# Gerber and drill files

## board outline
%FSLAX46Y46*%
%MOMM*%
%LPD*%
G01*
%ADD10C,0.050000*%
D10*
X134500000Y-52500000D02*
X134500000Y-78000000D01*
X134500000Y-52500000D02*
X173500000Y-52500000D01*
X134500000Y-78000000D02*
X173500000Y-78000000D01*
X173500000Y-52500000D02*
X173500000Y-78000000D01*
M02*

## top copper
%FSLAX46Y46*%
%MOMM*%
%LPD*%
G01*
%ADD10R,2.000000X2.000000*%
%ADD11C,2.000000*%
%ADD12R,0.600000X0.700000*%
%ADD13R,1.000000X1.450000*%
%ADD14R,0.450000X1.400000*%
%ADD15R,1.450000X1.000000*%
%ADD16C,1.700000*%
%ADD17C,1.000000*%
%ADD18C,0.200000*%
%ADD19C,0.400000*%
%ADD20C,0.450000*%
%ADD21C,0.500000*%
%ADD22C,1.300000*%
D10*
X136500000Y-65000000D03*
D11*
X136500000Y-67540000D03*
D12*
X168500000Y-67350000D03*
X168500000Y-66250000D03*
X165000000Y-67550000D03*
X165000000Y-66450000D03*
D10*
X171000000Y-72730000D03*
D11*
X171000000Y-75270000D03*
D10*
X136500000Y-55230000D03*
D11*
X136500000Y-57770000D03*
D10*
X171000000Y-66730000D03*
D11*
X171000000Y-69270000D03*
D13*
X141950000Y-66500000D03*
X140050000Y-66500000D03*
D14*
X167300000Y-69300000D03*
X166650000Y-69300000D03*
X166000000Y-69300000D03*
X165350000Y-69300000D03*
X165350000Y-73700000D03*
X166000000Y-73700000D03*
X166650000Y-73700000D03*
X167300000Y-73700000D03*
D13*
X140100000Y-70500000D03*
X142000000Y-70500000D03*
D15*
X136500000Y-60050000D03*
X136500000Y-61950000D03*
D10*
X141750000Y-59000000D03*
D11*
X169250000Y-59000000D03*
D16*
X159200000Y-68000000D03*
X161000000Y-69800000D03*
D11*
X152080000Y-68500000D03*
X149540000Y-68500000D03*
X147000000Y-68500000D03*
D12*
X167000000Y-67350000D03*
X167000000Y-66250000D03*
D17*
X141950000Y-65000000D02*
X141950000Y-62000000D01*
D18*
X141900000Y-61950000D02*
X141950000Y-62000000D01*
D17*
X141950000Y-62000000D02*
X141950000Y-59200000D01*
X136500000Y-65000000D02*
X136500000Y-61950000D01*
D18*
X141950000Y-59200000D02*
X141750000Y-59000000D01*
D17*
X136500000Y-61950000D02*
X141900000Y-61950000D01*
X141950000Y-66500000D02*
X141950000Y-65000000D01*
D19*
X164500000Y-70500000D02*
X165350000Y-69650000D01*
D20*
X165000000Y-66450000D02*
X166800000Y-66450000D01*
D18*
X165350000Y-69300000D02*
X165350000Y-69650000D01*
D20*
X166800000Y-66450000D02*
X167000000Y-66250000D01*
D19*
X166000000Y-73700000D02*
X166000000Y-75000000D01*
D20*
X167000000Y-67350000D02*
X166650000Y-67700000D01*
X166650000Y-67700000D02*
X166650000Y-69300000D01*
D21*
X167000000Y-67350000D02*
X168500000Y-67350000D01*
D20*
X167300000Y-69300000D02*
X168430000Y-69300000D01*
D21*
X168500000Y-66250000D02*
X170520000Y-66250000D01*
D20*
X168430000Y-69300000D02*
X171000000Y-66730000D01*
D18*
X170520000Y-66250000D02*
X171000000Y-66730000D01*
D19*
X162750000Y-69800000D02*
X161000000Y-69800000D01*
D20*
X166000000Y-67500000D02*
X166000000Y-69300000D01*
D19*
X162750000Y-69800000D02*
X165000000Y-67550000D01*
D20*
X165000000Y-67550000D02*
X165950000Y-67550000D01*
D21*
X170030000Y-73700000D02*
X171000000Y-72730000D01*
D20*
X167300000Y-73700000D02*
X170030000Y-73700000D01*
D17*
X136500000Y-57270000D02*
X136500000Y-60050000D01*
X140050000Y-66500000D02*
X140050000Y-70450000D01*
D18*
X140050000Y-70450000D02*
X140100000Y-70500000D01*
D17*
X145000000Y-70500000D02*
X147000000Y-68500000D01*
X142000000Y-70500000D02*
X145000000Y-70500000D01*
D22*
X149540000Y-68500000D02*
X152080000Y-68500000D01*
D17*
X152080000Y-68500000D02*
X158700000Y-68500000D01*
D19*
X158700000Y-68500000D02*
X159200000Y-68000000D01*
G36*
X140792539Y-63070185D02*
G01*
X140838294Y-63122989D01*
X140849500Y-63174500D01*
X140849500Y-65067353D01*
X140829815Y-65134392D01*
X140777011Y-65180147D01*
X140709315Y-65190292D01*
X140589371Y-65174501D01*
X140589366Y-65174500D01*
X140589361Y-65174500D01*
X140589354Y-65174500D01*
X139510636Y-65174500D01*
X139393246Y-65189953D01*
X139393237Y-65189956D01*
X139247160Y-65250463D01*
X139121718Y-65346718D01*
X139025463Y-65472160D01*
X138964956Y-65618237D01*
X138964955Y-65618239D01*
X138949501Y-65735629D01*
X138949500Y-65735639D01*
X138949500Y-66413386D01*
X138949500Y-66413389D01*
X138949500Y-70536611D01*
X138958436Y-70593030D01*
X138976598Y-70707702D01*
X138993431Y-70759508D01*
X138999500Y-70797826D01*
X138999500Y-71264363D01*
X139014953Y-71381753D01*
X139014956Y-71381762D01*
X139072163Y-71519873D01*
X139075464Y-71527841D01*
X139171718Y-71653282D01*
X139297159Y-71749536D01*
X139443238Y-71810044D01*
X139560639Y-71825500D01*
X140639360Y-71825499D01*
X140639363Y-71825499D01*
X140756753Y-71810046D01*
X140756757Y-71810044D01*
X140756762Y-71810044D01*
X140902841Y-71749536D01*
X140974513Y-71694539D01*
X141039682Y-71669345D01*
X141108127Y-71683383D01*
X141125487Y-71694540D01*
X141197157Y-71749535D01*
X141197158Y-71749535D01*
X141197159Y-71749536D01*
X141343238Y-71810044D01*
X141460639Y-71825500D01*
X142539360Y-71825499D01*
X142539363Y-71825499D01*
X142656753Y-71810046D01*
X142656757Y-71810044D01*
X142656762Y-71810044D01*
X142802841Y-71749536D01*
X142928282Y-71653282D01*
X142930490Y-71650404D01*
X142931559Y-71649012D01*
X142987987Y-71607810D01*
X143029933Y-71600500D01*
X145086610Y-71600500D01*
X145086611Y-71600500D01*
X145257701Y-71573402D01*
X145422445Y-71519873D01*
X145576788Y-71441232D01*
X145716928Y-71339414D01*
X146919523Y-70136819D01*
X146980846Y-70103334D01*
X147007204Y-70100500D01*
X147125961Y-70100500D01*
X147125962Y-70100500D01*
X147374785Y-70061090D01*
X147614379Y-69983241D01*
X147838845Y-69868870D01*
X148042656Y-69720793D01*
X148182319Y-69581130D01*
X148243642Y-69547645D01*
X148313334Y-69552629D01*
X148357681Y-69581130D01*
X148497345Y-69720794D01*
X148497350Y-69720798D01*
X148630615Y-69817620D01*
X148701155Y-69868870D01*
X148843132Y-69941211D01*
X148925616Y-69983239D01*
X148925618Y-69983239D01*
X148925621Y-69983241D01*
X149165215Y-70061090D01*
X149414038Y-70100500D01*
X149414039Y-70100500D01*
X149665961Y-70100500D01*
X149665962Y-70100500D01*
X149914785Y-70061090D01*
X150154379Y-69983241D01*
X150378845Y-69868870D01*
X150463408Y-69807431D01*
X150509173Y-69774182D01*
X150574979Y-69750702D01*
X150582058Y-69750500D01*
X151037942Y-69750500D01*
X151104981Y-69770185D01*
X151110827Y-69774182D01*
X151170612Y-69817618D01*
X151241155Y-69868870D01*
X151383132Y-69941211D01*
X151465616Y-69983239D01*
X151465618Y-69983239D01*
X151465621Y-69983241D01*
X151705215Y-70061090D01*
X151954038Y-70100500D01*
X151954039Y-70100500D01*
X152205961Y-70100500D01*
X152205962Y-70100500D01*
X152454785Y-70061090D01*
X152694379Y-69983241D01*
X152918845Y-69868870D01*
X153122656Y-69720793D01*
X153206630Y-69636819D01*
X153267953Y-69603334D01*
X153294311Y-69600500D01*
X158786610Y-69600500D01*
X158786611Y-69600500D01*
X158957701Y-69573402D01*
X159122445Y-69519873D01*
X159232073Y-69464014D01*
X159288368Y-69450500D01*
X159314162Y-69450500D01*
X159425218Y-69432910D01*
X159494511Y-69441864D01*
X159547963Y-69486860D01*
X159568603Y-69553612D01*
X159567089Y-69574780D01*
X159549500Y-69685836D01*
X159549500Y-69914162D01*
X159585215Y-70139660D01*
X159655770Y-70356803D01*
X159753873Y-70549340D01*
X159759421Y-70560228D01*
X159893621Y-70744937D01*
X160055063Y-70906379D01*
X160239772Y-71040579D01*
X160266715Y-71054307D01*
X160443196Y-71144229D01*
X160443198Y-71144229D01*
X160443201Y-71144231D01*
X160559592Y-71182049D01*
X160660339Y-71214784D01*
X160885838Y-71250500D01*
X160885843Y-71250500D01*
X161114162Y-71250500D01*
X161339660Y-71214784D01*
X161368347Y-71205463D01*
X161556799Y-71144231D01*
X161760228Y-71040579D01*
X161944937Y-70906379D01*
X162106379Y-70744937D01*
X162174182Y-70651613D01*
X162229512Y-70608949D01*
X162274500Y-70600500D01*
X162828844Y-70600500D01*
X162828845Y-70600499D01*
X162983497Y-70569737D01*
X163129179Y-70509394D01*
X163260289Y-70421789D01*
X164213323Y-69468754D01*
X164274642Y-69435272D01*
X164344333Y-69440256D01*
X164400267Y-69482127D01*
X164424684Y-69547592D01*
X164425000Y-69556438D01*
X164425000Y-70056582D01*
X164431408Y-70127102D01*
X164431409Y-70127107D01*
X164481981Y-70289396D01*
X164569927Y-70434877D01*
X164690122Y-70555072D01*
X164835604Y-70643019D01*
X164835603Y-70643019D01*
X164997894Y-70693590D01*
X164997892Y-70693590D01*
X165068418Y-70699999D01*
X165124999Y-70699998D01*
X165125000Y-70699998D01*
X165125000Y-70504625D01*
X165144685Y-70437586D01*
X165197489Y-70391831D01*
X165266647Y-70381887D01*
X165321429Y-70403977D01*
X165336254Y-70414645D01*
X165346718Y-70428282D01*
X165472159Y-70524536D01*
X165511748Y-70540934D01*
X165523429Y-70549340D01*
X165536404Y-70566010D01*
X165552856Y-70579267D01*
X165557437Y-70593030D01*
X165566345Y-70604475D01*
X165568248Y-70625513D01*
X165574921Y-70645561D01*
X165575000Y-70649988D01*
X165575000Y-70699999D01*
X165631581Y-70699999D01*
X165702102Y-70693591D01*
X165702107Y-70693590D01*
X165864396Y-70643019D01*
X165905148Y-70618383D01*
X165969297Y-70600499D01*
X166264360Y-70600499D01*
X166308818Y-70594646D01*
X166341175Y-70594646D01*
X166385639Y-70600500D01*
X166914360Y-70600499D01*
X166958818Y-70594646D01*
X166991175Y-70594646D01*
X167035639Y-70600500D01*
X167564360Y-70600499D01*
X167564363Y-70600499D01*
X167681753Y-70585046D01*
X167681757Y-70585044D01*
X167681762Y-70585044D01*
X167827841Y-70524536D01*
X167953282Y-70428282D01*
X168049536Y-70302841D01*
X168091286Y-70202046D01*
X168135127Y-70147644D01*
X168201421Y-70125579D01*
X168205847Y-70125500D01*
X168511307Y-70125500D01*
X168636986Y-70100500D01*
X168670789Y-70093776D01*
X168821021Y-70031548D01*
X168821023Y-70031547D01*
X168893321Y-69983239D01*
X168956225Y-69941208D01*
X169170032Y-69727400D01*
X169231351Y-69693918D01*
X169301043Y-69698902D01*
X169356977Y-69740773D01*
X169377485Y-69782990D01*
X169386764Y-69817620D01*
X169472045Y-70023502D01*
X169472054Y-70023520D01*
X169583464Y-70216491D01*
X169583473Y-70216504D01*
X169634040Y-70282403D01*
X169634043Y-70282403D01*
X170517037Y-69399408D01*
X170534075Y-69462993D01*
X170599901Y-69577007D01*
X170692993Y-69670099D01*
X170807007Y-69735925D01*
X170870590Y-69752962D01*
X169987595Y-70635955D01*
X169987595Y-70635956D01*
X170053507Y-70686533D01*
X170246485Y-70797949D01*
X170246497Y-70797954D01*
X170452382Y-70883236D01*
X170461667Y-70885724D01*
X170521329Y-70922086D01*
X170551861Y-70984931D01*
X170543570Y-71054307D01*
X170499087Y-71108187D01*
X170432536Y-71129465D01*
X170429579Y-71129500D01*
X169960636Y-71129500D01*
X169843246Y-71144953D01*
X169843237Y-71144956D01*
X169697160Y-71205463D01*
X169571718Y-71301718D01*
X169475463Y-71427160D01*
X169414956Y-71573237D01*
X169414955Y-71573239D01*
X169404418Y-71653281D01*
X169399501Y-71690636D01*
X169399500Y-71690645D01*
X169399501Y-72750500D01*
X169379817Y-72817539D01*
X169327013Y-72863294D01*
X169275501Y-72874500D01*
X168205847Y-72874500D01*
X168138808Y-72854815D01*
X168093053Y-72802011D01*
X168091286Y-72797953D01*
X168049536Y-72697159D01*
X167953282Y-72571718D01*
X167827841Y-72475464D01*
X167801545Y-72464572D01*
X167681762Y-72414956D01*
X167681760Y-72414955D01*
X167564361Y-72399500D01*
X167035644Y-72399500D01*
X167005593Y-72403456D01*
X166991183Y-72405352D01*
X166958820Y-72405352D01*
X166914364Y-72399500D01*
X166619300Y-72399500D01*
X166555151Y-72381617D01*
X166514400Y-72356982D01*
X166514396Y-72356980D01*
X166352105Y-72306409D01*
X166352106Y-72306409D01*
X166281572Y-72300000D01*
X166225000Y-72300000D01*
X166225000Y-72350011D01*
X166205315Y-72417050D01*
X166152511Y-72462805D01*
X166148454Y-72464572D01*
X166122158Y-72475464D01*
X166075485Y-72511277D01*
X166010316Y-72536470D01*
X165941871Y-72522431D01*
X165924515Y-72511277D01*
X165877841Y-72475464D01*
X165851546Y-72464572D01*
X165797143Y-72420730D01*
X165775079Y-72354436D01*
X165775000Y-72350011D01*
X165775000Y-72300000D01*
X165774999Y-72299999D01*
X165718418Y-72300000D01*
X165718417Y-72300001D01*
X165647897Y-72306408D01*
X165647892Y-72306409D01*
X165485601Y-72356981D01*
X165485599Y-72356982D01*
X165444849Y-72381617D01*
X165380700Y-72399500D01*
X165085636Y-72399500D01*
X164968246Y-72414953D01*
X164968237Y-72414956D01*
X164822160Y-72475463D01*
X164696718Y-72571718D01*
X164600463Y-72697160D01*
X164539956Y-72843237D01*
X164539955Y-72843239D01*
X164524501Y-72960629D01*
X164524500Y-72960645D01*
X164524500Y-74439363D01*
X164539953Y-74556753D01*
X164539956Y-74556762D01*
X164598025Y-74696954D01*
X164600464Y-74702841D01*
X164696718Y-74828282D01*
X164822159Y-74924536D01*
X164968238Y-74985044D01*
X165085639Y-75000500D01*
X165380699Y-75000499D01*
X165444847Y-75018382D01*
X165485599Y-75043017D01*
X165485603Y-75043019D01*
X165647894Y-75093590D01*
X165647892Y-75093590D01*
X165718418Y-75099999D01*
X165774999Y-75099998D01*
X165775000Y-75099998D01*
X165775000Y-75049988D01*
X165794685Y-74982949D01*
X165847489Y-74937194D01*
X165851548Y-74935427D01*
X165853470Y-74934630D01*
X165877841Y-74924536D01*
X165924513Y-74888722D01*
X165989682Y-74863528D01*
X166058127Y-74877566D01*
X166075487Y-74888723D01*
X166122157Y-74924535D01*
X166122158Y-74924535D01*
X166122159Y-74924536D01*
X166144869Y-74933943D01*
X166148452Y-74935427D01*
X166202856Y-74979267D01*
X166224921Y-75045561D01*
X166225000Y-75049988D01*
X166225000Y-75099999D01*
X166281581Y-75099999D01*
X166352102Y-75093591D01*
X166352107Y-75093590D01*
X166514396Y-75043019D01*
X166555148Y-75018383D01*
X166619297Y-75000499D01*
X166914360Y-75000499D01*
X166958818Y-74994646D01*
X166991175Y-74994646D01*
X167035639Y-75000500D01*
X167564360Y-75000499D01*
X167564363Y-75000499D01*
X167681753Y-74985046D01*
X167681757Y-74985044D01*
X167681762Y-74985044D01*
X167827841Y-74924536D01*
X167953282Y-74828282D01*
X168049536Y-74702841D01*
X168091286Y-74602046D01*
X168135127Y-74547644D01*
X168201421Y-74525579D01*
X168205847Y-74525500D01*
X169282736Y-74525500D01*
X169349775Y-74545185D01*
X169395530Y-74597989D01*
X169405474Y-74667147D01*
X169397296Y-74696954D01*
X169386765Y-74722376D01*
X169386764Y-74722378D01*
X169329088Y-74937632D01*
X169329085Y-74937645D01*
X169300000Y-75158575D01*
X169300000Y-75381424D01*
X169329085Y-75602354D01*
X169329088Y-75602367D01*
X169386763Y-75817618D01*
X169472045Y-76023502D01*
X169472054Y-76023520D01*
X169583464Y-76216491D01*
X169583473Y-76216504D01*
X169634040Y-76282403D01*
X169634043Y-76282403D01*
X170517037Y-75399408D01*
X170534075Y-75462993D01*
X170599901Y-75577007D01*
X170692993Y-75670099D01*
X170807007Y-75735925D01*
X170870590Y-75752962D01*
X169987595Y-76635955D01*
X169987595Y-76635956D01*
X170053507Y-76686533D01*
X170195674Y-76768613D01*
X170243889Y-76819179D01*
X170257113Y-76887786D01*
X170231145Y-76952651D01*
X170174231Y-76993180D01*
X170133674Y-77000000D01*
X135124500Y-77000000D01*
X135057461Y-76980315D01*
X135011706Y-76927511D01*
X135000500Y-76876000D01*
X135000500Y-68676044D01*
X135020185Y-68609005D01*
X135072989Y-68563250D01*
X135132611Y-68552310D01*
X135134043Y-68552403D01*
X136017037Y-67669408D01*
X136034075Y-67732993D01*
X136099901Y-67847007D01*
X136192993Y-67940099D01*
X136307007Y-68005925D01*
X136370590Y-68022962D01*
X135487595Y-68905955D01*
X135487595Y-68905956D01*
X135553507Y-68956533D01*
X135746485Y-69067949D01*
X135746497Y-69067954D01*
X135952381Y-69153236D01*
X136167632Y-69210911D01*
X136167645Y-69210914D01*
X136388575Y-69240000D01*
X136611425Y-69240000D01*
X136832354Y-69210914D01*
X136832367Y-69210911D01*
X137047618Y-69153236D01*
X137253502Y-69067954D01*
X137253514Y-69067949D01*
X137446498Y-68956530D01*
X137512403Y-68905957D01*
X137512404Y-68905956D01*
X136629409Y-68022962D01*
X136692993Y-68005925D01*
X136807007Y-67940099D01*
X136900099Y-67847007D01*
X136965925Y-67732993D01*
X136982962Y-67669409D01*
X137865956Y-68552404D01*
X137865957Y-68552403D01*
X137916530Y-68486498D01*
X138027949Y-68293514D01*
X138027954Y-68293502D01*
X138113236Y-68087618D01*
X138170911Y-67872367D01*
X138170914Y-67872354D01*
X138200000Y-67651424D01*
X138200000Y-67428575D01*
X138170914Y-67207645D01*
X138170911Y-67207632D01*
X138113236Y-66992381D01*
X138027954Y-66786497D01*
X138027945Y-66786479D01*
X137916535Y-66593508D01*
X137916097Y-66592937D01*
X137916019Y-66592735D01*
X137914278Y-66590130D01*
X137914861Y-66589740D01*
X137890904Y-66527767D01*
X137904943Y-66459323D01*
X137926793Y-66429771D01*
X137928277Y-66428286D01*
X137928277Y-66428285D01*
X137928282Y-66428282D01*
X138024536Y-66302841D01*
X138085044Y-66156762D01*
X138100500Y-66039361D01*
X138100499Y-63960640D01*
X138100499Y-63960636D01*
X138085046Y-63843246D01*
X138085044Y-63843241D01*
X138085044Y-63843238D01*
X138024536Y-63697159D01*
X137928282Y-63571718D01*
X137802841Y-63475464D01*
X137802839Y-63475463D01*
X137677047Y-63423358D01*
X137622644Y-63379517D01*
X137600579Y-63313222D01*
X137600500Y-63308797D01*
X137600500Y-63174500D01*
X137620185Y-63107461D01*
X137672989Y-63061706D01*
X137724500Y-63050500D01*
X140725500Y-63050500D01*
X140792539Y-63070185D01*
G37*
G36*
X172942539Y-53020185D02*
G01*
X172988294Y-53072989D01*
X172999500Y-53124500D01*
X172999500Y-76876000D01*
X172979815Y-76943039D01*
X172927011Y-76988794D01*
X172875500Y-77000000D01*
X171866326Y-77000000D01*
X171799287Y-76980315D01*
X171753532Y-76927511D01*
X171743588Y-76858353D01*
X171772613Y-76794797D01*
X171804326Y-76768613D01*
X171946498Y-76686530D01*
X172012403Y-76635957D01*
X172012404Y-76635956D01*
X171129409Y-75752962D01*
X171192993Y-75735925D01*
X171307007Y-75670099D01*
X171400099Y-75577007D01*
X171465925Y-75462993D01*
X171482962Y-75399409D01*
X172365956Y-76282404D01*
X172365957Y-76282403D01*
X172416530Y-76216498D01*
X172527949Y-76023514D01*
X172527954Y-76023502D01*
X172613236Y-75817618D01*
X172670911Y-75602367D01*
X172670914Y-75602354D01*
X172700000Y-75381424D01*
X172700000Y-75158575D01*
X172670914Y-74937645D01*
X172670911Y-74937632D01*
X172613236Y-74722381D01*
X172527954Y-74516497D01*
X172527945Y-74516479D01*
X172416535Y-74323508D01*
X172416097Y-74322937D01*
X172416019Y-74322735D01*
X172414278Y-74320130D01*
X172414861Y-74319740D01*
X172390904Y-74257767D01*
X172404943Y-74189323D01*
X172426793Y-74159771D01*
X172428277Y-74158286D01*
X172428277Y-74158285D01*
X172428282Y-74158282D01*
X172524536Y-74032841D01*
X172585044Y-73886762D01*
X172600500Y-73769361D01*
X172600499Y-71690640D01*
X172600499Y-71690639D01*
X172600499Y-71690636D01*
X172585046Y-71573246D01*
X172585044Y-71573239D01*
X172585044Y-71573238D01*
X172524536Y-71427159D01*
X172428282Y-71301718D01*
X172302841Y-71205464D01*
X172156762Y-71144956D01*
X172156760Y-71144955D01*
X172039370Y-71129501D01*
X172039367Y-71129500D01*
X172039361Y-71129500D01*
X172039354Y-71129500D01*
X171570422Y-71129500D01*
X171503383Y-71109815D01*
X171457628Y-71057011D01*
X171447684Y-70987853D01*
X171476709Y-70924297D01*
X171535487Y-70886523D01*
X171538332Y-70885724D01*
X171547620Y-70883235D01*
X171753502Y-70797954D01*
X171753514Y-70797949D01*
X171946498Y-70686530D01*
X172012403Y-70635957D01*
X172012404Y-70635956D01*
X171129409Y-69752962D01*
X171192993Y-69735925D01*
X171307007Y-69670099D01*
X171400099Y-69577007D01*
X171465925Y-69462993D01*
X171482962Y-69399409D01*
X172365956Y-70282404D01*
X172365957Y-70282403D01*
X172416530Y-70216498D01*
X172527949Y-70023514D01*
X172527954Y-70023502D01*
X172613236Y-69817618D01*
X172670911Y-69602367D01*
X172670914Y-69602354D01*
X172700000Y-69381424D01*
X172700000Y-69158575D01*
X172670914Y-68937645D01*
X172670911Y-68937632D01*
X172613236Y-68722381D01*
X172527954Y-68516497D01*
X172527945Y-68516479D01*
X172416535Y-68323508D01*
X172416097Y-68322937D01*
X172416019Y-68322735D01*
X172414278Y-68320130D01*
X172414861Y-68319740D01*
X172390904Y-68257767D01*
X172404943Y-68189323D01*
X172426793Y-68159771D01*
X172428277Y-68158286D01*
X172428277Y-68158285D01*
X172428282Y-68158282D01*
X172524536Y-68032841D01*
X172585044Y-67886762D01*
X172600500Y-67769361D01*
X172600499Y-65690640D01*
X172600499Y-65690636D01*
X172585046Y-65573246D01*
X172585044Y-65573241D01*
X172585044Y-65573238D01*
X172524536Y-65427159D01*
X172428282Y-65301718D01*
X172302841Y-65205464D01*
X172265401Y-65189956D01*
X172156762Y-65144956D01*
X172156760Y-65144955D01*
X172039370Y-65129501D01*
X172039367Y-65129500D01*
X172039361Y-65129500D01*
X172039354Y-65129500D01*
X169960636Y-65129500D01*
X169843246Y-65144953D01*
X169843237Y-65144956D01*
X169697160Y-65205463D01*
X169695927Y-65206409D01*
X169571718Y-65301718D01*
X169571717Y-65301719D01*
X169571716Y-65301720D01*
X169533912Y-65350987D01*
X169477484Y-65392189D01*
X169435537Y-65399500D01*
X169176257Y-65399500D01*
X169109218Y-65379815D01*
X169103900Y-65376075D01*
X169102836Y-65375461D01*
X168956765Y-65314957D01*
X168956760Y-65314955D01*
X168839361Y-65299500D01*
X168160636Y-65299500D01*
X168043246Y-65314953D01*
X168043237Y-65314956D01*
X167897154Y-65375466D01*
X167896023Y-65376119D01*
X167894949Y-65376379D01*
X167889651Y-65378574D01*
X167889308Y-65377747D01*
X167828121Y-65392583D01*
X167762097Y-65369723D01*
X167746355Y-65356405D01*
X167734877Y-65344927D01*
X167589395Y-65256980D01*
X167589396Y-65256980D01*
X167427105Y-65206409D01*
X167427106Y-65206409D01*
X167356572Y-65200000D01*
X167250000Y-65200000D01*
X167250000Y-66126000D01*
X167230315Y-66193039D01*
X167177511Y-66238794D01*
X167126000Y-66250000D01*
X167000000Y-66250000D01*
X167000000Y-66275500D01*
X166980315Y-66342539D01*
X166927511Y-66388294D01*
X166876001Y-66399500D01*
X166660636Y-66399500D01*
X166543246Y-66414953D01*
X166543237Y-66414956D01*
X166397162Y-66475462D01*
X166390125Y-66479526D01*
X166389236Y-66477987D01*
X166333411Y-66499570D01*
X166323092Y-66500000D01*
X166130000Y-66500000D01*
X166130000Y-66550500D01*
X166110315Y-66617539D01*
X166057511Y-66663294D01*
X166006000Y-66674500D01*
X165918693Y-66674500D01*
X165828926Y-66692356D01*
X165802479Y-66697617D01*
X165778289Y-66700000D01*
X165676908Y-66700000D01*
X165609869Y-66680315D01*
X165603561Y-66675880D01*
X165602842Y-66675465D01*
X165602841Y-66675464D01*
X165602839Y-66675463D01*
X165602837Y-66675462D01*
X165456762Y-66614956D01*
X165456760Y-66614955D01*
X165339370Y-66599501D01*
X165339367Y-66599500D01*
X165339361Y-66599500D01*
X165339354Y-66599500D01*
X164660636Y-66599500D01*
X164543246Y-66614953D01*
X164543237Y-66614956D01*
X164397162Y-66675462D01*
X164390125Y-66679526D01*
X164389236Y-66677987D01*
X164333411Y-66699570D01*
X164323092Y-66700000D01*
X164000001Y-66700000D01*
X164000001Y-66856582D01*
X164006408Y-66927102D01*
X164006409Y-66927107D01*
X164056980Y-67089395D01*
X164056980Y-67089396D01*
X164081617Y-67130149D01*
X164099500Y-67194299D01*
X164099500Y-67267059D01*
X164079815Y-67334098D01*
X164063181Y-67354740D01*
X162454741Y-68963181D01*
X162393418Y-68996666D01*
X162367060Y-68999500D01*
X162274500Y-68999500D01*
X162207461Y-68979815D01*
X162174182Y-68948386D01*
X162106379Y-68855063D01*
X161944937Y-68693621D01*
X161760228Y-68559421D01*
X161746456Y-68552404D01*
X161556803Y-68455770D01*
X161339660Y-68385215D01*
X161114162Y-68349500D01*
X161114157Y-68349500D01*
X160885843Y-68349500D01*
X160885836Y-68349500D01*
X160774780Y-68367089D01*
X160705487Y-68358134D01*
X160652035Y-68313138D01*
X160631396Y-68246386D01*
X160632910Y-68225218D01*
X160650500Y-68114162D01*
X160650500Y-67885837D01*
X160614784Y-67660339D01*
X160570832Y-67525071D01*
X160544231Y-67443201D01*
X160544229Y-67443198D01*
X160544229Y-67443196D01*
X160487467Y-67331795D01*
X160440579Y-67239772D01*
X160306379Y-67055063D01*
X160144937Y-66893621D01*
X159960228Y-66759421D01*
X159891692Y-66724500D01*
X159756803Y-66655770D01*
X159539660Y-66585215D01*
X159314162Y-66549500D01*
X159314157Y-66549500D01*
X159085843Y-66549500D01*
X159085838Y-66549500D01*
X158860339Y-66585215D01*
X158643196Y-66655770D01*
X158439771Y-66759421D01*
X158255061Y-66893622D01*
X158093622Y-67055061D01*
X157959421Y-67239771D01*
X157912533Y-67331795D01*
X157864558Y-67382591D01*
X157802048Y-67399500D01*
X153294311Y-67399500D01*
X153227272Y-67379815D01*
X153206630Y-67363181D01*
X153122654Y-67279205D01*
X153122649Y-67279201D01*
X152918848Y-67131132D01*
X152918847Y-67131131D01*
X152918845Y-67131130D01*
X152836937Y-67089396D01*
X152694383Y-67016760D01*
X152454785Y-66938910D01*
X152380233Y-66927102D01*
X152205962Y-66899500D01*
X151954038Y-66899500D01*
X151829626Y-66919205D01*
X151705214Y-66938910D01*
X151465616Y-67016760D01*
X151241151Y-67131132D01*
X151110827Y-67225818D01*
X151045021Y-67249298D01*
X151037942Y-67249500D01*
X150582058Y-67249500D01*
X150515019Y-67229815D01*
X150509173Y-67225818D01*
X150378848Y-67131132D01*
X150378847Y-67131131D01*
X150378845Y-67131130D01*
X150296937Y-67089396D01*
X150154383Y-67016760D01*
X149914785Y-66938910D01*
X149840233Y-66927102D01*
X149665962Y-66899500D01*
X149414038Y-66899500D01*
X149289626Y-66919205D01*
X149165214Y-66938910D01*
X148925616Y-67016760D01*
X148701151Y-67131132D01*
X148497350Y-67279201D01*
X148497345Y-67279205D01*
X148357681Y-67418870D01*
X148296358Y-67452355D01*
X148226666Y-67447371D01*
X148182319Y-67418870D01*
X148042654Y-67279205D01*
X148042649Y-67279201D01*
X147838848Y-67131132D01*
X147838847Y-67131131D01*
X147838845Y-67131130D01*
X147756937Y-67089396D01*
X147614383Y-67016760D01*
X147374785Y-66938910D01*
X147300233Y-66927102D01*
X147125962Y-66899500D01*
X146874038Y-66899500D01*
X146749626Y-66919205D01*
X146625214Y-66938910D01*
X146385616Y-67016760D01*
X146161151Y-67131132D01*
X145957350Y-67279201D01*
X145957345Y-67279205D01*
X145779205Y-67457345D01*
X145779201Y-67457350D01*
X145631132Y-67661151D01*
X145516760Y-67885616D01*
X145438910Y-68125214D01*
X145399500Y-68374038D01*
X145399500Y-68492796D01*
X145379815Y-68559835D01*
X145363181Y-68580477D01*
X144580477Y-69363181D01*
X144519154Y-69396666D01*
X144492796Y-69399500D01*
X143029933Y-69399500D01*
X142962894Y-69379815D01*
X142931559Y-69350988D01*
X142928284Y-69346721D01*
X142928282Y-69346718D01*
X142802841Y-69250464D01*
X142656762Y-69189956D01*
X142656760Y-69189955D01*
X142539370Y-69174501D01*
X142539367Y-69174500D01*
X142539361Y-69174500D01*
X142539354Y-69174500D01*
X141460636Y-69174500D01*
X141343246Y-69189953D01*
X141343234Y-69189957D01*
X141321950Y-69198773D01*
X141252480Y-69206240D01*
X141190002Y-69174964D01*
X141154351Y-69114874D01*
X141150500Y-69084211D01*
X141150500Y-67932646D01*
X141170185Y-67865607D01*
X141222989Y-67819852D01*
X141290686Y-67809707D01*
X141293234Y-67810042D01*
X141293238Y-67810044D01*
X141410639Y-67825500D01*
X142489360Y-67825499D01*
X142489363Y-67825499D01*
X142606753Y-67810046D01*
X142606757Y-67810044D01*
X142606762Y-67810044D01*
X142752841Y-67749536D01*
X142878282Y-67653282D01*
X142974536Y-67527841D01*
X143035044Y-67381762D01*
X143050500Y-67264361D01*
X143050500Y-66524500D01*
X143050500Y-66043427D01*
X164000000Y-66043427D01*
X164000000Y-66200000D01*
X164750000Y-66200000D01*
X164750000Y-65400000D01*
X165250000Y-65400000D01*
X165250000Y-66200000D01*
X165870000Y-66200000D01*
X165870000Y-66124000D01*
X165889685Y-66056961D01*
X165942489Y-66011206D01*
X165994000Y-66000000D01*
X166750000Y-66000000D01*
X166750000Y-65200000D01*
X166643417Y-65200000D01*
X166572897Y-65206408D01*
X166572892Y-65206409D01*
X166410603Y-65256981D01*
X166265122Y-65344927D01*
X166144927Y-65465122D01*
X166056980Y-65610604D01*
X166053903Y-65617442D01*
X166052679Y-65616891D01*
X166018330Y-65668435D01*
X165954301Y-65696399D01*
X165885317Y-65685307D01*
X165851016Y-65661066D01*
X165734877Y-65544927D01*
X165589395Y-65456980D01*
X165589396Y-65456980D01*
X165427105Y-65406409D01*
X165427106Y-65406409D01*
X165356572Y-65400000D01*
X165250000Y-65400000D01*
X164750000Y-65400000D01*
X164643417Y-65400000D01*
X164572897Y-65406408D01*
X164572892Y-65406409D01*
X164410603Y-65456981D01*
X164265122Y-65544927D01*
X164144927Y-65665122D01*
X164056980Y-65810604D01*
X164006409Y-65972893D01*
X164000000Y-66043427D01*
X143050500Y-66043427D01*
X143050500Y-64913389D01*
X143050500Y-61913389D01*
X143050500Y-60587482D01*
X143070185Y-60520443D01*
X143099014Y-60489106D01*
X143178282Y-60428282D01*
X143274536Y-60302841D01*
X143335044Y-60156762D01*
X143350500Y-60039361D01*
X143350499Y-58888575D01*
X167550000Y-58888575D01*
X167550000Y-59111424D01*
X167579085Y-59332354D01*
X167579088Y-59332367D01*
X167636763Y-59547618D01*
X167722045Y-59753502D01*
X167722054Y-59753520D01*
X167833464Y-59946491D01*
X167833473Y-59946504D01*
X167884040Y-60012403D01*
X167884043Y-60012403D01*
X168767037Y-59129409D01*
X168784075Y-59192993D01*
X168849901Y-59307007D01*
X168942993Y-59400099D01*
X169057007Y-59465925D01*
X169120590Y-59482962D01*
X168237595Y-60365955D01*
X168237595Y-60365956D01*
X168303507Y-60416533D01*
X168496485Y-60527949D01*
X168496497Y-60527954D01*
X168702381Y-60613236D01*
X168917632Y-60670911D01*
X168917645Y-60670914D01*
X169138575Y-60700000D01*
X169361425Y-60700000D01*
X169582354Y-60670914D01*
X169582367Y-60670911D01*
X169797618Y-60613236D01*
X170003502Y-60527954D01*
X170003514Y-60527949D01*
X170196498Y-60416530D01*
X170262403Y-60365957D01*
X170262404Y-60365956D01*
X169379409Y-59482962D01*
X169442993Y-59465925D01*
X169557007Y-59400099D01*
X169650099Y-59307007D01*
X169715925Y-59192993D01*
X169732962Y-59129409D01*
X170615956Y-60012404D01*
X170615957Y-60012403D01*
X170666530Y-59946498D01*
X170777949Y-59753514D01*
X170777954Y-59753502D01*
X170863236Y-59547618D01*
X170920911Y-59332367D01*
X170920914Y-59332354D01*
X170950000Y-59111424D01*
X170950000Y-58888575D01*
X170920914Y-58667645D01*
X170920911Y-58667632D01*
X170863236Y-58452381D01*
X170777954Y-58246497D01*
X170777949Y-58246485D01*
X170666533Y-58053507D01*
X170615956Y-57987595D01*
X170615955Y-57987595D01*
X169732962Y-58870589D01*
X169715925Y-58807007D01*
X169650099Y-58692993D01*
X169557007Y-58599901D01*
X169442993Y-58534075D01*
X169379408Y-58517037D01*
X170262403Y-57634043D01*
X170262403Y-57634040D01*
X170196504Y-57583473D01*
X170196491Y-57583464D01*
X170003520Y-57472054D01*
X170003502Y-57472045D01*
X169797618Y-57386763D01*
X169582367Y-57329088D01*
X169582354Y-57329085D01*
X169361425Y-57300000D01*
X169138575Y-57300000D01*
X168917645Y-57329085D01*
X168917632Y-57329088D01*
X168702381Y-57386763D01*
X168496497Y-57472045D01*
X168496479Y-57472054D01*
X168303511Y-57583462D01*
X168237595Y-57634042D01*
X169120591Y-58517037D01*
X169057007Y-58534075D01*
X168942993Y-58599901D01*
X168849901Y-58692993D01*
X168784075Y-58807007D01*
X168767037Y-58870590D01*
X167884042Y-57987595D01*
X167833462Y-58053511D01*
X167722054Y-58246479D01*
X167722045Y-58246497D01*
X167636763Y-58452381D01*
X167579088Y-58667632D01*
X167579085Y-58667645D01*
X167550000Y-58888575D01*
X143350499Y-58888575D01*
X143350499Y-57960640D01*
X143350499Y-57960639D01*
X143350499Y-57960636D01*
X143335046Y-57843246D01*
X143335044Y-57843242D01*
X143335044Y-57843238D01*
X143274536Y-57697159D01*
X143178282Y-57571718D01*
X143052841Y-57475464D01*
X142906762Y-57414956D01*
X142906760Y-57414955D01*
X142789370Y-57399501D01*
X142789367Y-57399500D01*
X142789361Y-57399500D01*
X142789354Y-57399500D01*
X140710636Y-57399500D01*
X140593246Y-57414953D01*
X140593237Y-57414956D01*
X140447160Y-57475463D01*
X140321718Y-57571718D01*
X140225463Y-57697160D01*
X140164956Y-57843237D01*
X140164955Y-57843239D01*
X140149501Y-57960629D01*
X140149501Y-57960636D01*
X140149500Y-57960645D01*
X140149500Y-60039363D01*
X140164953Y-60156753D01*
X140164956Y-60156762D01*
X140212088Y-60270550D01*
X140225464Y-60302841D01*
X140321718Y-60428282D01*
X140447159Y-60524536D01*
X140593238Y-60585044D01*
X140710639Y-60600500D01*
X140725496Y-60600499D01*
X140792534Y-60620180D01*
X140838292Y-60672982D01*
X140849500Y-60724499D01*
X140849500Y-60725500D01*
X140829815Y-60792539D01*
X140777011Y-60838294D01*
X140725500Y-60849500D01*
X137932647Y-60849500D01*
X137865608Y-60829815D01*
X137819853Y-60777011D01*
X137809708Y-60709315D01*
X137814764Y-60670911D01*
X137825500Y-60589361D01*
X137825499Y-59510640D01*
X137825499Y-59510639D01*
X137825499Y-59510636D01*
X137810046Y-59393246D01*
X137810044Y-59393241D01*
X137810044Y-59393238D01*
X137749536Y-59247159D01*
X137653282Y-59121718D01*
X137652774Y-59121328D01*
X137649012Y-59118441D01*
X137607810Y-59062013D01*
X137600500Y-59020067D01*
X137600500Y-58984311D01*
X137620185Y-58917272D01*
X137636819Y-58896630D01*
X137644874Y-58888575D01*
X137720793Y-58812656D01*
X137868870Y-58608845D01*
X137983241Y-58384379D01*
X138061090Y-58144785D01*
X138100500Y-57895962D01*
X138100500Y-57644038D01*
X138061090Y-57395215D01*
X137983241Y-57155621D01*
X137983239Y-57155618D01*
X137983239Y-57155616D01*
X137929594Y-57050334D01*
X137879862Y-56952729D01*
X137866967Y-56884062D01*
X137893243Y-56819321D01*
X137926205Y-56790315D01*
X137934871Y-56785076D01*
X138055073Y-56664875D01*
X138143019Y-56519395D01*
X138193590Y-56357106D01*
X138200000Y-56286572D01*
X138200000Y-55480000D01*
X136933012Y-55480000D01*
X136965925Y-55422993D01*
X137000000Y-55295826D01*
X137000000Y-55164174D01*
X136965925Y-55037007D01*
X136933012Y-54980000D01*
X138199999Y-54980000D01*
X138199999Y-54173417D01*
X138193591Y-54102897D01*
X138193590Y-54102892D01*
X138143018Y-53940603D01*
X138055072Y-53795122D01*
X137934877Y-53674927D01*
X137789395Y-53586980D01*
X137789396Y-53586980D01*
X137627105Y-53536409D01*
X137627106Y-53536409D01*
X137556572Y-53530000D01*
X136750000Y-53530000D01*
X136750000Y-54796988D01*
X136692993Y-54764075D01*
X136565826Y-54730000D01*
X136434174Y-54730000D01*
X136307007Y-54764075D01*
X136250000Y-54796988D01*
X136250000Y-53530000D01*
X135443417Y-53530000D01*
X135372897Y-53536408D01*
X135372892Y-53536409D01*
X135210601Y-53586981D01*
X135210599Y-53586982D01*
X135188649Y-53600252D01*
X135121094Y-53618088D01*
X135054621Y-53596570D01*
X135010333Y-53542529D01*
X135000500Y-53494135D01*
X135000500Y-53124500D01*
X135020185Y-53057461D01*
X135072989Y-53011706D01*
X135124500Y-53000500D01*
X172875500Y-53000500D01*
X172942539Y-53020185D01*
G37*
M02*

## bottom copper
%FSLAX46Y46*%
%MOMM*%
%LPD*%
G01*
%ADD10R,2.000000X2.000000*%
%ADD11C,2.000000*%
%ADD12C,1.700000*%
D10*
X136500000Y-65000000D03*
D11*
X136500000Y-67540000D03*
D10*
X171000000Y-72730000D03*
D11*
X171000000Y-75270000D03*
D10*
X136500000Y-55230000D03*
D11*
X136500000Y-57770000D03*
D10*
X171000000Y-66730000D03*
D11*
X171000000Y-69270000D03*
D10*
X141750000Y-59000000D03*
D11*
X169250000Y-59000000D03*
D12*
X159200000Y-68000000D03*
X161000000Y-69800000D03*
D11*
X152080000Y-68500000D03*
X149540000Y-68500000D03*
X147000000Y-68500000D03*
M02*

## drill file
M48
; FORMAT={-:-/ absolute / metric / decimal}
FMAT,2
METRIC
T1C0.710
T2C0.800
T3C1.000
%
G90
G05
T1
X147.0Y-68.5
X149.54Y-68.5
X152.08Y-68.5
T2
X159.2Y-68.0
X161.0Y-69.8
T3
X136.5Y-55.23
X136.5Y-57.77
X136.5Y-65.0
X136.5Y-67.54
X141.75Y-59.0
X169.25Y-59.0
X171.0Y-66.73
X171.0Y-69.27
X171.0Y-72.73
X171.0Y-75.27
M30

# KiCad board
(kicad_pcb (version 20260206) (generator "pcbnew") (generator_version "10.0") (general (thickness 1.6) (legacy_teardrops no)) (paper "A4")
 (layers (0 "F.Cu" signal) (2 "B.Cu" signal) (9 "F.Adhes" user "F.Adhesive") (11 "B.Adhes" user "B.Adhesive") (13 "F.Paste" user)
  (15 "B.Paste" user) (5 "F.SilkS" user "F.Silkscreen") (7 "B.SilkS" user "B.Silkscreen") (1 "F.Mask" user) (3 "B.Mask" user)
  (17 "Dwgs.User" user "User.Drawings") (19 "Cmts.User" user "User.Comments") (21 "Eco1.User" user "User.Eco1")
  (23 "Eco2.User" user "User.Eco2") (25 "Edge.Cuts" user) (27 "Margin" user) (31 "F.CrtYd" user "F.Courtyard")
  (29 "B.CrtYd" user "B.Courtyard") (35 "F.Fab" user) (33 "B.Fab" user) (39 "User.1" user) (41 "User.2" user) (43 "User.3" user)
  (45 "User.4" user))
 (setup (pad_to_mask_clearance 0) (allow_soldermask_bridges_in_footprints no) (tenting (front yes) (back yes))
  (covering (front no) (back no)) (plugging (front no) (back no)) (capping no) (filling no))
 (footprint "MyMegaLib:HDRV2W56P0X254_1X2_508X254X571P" (layer "F.Cu") (at 136.5 65 -90)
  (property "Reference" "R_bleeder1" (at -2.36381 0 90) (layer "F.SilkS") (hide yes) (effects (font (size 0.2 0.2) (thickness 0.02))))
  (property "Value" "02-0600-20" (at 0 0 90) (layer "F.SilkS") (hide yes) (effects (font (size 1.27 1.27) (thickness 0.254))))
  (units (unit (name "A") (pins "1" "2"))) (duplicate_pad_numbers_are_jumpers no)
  (pad "1" thru_hole rect (at 0 0 270) (size 2 2) (drill 1) (layers "*.Cu" "*.Mask") (remove_unused_layers no)
   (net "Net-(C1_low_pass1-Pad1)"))
  (pad "2" thru_hole circle (at 2.54 0 270) (size 2 2) (drill 1) (layers "*.Cu" "*.Mask") (remove_unused_layers no) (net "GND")))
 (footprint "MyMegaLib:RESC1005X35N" (layer "F.Cu") (at 168.5 66.8 90)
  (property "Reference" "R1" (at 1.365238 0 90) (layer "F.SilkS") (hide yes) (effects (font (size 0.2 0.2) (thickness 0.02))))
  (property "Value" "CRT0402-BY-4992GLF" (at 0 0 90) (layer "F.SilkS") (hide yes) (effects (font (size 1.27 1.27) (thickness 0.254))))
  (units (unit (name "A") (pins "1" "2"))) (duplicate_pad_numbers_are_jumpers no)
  (pad "1" smd rect (at -0.55 0 180) (size 0.6 0.7) (layers "F.Cu" "F.Mask" "F.Paste") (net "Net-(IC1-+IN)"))
  (pad "2" smd rect (at 0.55 0 180) (size 0.6 0.7) (layers "F.Cu" "F.Mask" "F.Paste") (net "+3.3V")))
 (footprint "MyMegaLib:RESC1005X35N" (layer "F.Cu") (at 165 67 90)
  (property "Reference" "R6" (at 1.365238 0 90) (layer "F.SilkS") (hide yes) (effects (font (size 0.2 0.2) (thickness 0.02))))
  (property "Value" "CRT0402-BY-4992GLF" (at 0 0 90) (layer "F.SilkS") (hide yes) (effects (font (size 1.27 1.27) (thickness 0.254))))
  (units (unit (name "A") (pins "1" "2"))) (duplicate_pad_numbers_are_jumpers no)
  (pad "1" smd rect (at -0.55 0 180) (size 0.6 0.7) (layers "F.Cu" "F.Mask" "F.Paste") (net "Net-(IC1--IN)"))
  (pad "2" smd rect (at 0.55 0 180) (size 0.6 0.7) (layers "F.Cu" "F.Mask" "F.Paste") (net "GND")))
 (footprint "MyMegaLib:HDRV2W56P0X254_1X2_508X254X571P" (layer "F.Cu") (at 171 72.73 -90)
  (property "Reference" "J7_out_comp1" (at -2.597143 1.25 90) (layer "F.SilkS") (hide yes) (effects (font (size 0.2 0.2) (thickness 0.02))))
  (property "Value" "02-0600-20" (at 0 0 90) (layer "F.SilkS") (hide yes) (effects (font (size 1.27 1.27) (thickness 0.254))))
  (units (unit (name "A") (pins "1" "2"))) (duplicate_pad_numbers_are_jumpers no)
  (pad "1" thru_hole rect (at 0 0 270) (size 2 2) (drill 1) (layers "*.Cu" "*.Mask") (remove_unused_layers no) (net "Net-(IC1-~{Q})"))
  (pad "2" thru_hole circle (at 2.54 0 270) (size 2 2) (drill 1) (layers "*.Cu" "*.Mask") (remove_unused_layers no) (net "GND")))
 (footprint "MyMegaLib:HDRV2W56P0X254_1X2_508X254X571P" (layer "F.Cu") (at 136.5 55.23 -90)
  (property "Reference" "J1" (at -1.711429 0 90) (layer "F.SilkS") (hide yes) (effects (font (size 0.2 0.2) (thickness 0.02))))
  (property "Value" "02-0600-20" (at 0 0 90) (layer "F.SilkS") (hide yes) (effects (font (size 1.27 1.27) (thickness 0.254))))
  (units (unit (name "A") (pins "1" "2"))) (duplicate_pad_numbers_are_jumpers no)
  (pad "1" thru_hole rect (at 0 0 270) (size 2 2) (drill 1) (layers "*.Cu" "*.Mask") (remove_unused_layers no) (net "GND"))
  (pad "2" thru_hole circle (at 2.54 0 270) (size 2 2) (drill 1) (layers "*.Cu" "*.Mask") (remove_unused_layers no) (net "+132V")))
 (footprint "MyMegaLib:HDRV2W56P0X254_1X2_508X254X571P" (layer "F.Cu") (at 171 66.73 -90)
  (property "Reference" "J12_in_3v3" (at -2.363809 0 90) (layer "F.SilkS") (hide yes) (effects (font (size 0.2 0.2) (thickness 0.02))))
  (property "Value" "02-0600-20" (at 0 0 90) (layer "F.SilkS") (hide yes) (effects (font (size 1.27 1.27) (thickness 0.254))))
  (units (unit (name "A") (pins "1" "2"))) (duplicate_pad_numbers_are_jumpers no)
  (pad "1" thru_hole rect (at 0 0 270) (size 2 2) (drill 1) (layers "*.Cu" "*.Mask") (remove_unused_layers no) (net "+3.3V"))
  (pad "2" thru_hole circle (at 2.54 0 270) (size 2 2) (drill 1) (layers "*.Cu" "*.Mask") (remove_unused_layers no) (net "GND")))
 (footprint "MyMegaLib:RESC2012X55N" (layer "F.Cu") (at 141 66.5 180)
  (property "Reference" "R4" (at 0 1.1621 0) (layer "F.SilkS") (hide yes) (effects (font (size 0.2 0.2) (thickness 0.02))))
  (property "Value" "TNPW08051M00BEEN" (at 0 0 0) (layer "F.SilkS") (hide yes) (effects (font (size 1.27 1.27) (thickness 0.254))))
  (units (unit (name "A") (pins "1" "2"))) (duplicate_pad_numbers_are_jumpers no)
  (pad "1" smd rect (at -0.95 0 180) (size 1 1.45) (layers "F.Cu" "F.Mask" "F.Paste") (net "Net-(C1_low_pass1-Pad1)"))
  (pad "2" smd rect (at 0.95 0 180) (size 1 1.45) (layers "F.Cu" "F.Mask" "F.Paste") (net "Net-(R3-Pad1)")))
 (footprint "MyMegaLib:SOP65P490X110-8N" (layer "F.Cu") (at 166.325 71.5 -90)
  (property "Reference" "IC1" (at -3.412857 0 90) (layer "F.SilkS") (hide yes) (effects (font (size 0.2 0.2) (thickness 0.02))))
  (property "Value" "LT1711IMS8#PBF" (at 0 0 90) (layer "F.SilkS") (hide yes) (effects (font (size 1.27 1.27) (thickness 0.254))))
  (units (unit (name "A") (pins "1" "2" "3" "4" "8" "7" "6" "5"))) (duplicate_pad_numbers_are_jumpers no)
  (pad "1" smd rect (at -2.2 -0.975) (size 0.45 1.4) (layers "F.Cu" "F.Mask" "F.Paste") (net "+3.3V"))
  (pad "2" smd rect (at -2.2 -0.325) (size 0.45 1.4) (layers "F.Cu" "F.Mask" "F.Paste") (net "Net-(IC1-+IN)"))
  (pad "3" smd rect (at -2.2 0.325) (size 0.45 1.4) (layers "F.Cu" "F.Mask" "F.Paste") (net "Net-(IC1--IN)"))
  (pad "4" smd rect (at -2.2 0.975) (size 0.45 1.4) (layers "F.Cu" "F.Mask" "F.Paste") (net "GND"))
  (pad "5" smd rect (at 2.2 0.975) (size 0.45 1.4) (layers "F.Cu" "F.Mask" "F.Paste") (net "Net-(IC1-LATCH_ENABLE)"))
  (pad "6" smd rect (at 2.2 0.325) (size 0.45 1.4) (layers "F.Cu" "F.Mask" "F.Paste") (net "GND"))
  (pad "7" smd rect (at 2.2 -0.325) (size 0.45 1.4) (layers "F.Cu" "F.Mask" "F.Paste") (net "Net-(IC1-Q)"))
  (pad "8" smd rect (at 2.2 -0.975) (size 0.45 1.4) (layers "F.Cu" "F.Mask" "F.Paste") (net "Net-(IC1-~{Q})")))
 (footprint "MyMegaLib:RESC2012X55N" (layer "F.Cu") (at 141.05 70.5)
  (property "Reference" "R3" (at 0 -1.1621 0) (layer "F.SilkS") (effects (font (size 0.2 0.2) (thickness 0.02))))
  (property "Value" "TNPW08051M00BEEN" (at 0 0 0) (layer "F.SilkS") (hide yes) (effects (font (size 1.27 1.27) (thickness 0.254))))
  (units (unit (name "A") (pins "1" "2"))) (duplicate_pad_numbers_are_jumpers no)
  (pad "1" smd rect (at -0.95 0) (size 1 1.45) (layers "F.Cu" "F.Mask" "F.Paste") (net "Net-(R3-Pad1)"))
  (pad "2" smd rect (at 0.95 0) (size 1 1.45) (layers "F.Cu" "F.Mask" "F.Paste") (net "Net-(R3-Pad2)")))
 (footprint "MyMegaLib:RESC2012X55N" (layer "F.Cu") (at 136.5 61 -90)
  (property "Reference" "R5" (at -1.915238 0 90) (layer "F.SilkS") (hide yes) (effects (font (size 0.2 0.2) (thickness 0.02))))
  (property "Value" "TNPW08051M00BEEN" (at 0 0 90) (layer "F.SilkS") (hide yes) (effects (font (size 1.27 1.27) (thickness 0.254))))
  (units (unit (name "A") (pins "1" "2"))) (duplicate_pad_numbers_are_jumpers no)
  (pad "1" smd rect (at -0.95 0 270) (size 1 1.45) (layers "F.Cu" "F.Mask" "F.Paste") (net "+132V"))
  (pad "2" smd rect (at 0.95 0 270) (size 1 1.45) (layers "F.Cu" "F.Mask" "F.Paste") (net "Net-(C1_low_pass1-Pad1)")))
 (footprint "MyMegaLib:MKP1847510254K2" (layer "F.Cu") (at 141.75 59)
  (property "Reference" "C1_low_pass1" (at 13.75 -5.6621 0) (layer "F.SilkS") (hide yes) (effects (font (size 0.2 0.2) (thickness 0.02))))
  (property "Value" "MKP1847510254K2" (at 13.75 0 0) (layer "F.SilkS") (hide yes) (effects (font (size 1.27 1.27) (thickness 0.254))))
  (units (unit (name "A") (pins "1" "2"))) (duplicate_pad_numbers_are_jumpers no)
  (pad "1" thru_hole rect (at 0 0) (size 2 2) (drill 1) (layers "*.Cu" "*.Mask") (remove_unused_layers no) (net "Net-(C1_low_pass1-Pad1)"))
  (pad "2" thru_hole circle (at 27.5 0) (size 2 2) (drill 1) (layers "*.Cu" "*.Mask") (remove_unused_layers no) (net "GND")))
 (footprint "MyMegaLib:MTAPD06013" (layer "F.Cu") (at 160.1 68.9 -90)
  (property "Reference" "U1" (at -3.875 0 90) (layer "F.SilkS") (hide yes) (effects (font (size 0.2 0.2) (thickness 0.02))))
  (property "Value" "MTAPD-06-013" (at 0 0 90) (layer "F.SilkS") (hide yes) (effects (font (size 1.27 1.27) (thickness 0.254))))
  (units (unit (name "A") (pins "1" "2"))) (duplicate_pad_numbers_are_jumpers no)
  (pad "1" thru_hole circle (at -0.9 0.9 270) (size 1.7 1.7) (drill 0.8) (layers "*.Cu" "*.Mask") (remove_unused_layers no)
   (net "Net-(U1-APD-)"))
  (pad "2" thru_hole circle (at 0.9 -0.9 270) (size 1.7 1.7) (drill 0.8) (layers "*.Cu" "*.Mask") (remove_unused_layers no)
   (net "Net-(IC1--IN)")))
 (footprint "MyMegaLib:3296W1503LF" (layer "F.Cu") (at 152.08 68.5)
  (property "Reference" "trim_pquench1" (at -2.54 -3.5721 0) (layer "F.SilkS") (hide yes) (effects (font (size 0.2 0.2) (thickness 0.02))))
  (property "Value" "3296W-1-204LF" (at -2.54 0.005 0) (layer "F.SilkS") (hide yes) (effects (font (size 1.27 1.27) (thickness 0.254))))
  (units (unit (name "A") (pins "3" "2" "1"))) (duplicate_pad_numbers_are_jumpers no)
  (pad "1" thru_hole circle (at 0 0) (size 2 2) (drill 0.71) (layers "*.Cu" "*.Mask") (remove_unused_layers no) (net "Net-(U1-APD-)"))
  (pad "2" thru_hole circle (at -2.54 0) (size 2 2) (drill 0.71) (layers "*.Cu" "*.Mask") (remove_unused_layers no) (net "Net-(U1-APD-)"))
  (pad "3" thru_hole circle (at -5.08 0) (size 2 2) (drill 0.71) (layers "*.Cu" "*.Mask") (remove_unused_layers no) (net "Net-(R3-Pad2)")))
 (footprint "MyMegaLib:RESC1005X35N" (layer "F.Cu") (at 167 66.8 90)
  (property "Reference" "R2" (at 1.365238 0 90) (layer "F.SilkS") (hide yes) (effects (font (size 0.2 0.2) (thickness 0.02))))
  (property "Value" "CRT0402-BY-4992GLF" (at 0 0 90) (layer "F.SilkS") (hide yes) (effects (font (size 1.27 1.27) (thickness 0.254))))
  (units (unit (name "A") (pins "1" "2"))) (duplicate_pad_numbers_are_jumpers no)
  (pad "1" smd rect (at -0.55 0 180) (size 0.6 0.7) (layers "F.Cu" "F.Mask" "F.Paste") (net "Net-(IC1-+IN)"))
  (pad "2" smd rect (at 0.55 0 180) (size 0.6 0.7) (layers "F.Cu" "F.Mask" "F.Paste") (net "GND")))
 (gr_line (start 134.5 52.5) (end 134.5 78) (stroke (width 0.05) (type default)) (layer "Edge.Cuts"))
 (gr_line (start 134.5 52.5) (end 173.5 52.5) (stroke (width 0.05) (type default)) (layer "Edge.Cuts"))
 (gr_line (start 134.5 78) (end 173.5 78) (stroke (width 0.05) (type default)) (layer "Edge.Cuts"))
 (gr_line (start 173.5 52.5) (end 173.5 78) (stroke (width 0.05) (type default)) (layer "Edge.Cuts"))
 (segment (start 141.95 65) (end 141.95 62) (width 1) (layer "F.Cu") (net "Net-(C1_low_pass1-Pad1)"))
 (segment (start 141.9 61.95) (end 141.95 62) (width 0.2) (layer "F.Cu") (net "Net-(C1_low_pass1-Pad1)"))
 (segment (start 141.95 62) (end 141.95 59.2) (width 1) (layer "F.Cu") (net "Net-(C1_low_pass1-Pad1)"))
 (segment (start 136.5 65) (end 136.5 61.95) (width 1) (layer "F.Cu") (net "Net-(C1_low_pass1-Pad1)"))
 (segment (start 141.95 59.2) (end 141.75 59) (width 0.2) (layer "F.Cu") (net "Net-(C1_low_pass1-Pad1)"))
 (segment (start 136.5 61.95) (end 141.9 61.95) (width 1) (layer "F.Cu") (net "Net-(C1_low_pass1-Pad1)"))
 (segment (start 141.95 66.5) (end 141.95 65) (width 1) (layer "F.Cu") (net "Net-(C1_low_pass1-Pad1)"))
 (segment (start 164.5 70.5) (end 165.35 69.65) (width 0.4) (layer "F.Cu") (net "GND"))
 (segment (start 165 66.45) (end 166.8 66.45) (width 0.45) (layer "F.Cu") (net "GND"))
 (segment (start 165.35 69.3) (end 165.35 69.65) (width 0.2) (layer "F.Cu") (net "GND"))
 (segment (start 166.8 66.45) (end 167 66.25) (width 0.45) (layer "F.Cu") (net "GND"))
 (segment (start 166 73.7) (end 166 75) (width 0.4) (layer "F.Cu") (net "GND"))
 (segment (start 167 67.35) (end 166.65 67.7) (width 0.45) (layer "F.Cu") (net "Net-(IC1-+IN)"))
 (segment (start 166.65 67.7) (end 166.65 69.3) (width 0.45) (layer "F.Cu") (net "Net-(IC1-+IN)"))
 (segment (start 167 67.35) (end 168.5 67.35) (width 0.5) (layer "F.Cu") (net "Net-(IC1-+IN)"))
 (segment (start 167.3 69.3) (end 168.43 69.3) (width 0.45) (layer "F.Cu") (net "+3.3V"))
 (segment (start 168.5 66.25) (end 170.52 66.25) (width 0.5) (layer "F.Cu") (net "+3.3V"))
 (segment (start 168.43 69.3) (end 171 66.73) (width 0.45) (layer "F.Cu") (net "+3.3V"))
 (segment (start 170.52 66.25) (end 171 66.73) (width 0.2) (layer "F.Cu") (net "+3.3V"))
 (segment (start 162.75 69.8) (end 161 69.8) (width 0.4) (layer "F.Cu") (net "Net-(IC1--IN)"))
 (segment (start 166 67.5) (end 166 69.3) (width 0.45) (layer "F.Cu") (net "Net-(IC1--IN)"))
 (segment (start 162.75 69.8) (end 165 67.55) (width 0.4) (layer "F.Cu") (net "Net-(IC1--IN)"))
 (segment (start 165 67.55) (end 165.95 67.55) (width 0.45) (layer "F.Cu") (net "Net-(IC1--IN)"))
 (segment (start 170.03 73.7) (end 171 72.73) (width 0.5) (layer "F.Cu") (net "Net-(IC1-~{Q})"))
 (segment (start 167.3 73.7) (end 170.03 73.7) (width 0.45) (layer "F.Cu") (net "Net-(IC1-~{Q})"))
 (segment (start 136.5 57.27) (end 136.5 60.05) (width 1) (layer "F.Cu") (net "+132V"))
 (segment (start 140.05 66.5) (end 140.05 70.45) (width 1) (layer "F.Cu") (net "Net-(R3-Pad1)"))
 (segment (start 140.05 70.45) (end 140.1 70.5) (width 0.2) (layer "F.Cu") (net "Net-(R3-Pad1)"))
 (segment (start 145 70.5) (end 147 68.5) (width 1) (layer "F.Cu") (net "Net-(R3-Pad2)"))
 (segment (start 142 70.5) (end 145 70.5) (width 1) (layer "F.Cu") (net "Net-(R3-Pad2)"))
 (segment (start 149.54 68.5) (end 152.08 68.5) (width 1.3) (layer "F.Cu") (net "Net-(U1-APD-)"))
 (segment (start 152.08 68.5) (end 158.7 68.5) (width 1) (layer "F.Cu") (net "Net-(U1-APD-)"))
 (segment (start 158.7 68.5) (end 159.2 68) (width 0.4) (layer "F.Cu") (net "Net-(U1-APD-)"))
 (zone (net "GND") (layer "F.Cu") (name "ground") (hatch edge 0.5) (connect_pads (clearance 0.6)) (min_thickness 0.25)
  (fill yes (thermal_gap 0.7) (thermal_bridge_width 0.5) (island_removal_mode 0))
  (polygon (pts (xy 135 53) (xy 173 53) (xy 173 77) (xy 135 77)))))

